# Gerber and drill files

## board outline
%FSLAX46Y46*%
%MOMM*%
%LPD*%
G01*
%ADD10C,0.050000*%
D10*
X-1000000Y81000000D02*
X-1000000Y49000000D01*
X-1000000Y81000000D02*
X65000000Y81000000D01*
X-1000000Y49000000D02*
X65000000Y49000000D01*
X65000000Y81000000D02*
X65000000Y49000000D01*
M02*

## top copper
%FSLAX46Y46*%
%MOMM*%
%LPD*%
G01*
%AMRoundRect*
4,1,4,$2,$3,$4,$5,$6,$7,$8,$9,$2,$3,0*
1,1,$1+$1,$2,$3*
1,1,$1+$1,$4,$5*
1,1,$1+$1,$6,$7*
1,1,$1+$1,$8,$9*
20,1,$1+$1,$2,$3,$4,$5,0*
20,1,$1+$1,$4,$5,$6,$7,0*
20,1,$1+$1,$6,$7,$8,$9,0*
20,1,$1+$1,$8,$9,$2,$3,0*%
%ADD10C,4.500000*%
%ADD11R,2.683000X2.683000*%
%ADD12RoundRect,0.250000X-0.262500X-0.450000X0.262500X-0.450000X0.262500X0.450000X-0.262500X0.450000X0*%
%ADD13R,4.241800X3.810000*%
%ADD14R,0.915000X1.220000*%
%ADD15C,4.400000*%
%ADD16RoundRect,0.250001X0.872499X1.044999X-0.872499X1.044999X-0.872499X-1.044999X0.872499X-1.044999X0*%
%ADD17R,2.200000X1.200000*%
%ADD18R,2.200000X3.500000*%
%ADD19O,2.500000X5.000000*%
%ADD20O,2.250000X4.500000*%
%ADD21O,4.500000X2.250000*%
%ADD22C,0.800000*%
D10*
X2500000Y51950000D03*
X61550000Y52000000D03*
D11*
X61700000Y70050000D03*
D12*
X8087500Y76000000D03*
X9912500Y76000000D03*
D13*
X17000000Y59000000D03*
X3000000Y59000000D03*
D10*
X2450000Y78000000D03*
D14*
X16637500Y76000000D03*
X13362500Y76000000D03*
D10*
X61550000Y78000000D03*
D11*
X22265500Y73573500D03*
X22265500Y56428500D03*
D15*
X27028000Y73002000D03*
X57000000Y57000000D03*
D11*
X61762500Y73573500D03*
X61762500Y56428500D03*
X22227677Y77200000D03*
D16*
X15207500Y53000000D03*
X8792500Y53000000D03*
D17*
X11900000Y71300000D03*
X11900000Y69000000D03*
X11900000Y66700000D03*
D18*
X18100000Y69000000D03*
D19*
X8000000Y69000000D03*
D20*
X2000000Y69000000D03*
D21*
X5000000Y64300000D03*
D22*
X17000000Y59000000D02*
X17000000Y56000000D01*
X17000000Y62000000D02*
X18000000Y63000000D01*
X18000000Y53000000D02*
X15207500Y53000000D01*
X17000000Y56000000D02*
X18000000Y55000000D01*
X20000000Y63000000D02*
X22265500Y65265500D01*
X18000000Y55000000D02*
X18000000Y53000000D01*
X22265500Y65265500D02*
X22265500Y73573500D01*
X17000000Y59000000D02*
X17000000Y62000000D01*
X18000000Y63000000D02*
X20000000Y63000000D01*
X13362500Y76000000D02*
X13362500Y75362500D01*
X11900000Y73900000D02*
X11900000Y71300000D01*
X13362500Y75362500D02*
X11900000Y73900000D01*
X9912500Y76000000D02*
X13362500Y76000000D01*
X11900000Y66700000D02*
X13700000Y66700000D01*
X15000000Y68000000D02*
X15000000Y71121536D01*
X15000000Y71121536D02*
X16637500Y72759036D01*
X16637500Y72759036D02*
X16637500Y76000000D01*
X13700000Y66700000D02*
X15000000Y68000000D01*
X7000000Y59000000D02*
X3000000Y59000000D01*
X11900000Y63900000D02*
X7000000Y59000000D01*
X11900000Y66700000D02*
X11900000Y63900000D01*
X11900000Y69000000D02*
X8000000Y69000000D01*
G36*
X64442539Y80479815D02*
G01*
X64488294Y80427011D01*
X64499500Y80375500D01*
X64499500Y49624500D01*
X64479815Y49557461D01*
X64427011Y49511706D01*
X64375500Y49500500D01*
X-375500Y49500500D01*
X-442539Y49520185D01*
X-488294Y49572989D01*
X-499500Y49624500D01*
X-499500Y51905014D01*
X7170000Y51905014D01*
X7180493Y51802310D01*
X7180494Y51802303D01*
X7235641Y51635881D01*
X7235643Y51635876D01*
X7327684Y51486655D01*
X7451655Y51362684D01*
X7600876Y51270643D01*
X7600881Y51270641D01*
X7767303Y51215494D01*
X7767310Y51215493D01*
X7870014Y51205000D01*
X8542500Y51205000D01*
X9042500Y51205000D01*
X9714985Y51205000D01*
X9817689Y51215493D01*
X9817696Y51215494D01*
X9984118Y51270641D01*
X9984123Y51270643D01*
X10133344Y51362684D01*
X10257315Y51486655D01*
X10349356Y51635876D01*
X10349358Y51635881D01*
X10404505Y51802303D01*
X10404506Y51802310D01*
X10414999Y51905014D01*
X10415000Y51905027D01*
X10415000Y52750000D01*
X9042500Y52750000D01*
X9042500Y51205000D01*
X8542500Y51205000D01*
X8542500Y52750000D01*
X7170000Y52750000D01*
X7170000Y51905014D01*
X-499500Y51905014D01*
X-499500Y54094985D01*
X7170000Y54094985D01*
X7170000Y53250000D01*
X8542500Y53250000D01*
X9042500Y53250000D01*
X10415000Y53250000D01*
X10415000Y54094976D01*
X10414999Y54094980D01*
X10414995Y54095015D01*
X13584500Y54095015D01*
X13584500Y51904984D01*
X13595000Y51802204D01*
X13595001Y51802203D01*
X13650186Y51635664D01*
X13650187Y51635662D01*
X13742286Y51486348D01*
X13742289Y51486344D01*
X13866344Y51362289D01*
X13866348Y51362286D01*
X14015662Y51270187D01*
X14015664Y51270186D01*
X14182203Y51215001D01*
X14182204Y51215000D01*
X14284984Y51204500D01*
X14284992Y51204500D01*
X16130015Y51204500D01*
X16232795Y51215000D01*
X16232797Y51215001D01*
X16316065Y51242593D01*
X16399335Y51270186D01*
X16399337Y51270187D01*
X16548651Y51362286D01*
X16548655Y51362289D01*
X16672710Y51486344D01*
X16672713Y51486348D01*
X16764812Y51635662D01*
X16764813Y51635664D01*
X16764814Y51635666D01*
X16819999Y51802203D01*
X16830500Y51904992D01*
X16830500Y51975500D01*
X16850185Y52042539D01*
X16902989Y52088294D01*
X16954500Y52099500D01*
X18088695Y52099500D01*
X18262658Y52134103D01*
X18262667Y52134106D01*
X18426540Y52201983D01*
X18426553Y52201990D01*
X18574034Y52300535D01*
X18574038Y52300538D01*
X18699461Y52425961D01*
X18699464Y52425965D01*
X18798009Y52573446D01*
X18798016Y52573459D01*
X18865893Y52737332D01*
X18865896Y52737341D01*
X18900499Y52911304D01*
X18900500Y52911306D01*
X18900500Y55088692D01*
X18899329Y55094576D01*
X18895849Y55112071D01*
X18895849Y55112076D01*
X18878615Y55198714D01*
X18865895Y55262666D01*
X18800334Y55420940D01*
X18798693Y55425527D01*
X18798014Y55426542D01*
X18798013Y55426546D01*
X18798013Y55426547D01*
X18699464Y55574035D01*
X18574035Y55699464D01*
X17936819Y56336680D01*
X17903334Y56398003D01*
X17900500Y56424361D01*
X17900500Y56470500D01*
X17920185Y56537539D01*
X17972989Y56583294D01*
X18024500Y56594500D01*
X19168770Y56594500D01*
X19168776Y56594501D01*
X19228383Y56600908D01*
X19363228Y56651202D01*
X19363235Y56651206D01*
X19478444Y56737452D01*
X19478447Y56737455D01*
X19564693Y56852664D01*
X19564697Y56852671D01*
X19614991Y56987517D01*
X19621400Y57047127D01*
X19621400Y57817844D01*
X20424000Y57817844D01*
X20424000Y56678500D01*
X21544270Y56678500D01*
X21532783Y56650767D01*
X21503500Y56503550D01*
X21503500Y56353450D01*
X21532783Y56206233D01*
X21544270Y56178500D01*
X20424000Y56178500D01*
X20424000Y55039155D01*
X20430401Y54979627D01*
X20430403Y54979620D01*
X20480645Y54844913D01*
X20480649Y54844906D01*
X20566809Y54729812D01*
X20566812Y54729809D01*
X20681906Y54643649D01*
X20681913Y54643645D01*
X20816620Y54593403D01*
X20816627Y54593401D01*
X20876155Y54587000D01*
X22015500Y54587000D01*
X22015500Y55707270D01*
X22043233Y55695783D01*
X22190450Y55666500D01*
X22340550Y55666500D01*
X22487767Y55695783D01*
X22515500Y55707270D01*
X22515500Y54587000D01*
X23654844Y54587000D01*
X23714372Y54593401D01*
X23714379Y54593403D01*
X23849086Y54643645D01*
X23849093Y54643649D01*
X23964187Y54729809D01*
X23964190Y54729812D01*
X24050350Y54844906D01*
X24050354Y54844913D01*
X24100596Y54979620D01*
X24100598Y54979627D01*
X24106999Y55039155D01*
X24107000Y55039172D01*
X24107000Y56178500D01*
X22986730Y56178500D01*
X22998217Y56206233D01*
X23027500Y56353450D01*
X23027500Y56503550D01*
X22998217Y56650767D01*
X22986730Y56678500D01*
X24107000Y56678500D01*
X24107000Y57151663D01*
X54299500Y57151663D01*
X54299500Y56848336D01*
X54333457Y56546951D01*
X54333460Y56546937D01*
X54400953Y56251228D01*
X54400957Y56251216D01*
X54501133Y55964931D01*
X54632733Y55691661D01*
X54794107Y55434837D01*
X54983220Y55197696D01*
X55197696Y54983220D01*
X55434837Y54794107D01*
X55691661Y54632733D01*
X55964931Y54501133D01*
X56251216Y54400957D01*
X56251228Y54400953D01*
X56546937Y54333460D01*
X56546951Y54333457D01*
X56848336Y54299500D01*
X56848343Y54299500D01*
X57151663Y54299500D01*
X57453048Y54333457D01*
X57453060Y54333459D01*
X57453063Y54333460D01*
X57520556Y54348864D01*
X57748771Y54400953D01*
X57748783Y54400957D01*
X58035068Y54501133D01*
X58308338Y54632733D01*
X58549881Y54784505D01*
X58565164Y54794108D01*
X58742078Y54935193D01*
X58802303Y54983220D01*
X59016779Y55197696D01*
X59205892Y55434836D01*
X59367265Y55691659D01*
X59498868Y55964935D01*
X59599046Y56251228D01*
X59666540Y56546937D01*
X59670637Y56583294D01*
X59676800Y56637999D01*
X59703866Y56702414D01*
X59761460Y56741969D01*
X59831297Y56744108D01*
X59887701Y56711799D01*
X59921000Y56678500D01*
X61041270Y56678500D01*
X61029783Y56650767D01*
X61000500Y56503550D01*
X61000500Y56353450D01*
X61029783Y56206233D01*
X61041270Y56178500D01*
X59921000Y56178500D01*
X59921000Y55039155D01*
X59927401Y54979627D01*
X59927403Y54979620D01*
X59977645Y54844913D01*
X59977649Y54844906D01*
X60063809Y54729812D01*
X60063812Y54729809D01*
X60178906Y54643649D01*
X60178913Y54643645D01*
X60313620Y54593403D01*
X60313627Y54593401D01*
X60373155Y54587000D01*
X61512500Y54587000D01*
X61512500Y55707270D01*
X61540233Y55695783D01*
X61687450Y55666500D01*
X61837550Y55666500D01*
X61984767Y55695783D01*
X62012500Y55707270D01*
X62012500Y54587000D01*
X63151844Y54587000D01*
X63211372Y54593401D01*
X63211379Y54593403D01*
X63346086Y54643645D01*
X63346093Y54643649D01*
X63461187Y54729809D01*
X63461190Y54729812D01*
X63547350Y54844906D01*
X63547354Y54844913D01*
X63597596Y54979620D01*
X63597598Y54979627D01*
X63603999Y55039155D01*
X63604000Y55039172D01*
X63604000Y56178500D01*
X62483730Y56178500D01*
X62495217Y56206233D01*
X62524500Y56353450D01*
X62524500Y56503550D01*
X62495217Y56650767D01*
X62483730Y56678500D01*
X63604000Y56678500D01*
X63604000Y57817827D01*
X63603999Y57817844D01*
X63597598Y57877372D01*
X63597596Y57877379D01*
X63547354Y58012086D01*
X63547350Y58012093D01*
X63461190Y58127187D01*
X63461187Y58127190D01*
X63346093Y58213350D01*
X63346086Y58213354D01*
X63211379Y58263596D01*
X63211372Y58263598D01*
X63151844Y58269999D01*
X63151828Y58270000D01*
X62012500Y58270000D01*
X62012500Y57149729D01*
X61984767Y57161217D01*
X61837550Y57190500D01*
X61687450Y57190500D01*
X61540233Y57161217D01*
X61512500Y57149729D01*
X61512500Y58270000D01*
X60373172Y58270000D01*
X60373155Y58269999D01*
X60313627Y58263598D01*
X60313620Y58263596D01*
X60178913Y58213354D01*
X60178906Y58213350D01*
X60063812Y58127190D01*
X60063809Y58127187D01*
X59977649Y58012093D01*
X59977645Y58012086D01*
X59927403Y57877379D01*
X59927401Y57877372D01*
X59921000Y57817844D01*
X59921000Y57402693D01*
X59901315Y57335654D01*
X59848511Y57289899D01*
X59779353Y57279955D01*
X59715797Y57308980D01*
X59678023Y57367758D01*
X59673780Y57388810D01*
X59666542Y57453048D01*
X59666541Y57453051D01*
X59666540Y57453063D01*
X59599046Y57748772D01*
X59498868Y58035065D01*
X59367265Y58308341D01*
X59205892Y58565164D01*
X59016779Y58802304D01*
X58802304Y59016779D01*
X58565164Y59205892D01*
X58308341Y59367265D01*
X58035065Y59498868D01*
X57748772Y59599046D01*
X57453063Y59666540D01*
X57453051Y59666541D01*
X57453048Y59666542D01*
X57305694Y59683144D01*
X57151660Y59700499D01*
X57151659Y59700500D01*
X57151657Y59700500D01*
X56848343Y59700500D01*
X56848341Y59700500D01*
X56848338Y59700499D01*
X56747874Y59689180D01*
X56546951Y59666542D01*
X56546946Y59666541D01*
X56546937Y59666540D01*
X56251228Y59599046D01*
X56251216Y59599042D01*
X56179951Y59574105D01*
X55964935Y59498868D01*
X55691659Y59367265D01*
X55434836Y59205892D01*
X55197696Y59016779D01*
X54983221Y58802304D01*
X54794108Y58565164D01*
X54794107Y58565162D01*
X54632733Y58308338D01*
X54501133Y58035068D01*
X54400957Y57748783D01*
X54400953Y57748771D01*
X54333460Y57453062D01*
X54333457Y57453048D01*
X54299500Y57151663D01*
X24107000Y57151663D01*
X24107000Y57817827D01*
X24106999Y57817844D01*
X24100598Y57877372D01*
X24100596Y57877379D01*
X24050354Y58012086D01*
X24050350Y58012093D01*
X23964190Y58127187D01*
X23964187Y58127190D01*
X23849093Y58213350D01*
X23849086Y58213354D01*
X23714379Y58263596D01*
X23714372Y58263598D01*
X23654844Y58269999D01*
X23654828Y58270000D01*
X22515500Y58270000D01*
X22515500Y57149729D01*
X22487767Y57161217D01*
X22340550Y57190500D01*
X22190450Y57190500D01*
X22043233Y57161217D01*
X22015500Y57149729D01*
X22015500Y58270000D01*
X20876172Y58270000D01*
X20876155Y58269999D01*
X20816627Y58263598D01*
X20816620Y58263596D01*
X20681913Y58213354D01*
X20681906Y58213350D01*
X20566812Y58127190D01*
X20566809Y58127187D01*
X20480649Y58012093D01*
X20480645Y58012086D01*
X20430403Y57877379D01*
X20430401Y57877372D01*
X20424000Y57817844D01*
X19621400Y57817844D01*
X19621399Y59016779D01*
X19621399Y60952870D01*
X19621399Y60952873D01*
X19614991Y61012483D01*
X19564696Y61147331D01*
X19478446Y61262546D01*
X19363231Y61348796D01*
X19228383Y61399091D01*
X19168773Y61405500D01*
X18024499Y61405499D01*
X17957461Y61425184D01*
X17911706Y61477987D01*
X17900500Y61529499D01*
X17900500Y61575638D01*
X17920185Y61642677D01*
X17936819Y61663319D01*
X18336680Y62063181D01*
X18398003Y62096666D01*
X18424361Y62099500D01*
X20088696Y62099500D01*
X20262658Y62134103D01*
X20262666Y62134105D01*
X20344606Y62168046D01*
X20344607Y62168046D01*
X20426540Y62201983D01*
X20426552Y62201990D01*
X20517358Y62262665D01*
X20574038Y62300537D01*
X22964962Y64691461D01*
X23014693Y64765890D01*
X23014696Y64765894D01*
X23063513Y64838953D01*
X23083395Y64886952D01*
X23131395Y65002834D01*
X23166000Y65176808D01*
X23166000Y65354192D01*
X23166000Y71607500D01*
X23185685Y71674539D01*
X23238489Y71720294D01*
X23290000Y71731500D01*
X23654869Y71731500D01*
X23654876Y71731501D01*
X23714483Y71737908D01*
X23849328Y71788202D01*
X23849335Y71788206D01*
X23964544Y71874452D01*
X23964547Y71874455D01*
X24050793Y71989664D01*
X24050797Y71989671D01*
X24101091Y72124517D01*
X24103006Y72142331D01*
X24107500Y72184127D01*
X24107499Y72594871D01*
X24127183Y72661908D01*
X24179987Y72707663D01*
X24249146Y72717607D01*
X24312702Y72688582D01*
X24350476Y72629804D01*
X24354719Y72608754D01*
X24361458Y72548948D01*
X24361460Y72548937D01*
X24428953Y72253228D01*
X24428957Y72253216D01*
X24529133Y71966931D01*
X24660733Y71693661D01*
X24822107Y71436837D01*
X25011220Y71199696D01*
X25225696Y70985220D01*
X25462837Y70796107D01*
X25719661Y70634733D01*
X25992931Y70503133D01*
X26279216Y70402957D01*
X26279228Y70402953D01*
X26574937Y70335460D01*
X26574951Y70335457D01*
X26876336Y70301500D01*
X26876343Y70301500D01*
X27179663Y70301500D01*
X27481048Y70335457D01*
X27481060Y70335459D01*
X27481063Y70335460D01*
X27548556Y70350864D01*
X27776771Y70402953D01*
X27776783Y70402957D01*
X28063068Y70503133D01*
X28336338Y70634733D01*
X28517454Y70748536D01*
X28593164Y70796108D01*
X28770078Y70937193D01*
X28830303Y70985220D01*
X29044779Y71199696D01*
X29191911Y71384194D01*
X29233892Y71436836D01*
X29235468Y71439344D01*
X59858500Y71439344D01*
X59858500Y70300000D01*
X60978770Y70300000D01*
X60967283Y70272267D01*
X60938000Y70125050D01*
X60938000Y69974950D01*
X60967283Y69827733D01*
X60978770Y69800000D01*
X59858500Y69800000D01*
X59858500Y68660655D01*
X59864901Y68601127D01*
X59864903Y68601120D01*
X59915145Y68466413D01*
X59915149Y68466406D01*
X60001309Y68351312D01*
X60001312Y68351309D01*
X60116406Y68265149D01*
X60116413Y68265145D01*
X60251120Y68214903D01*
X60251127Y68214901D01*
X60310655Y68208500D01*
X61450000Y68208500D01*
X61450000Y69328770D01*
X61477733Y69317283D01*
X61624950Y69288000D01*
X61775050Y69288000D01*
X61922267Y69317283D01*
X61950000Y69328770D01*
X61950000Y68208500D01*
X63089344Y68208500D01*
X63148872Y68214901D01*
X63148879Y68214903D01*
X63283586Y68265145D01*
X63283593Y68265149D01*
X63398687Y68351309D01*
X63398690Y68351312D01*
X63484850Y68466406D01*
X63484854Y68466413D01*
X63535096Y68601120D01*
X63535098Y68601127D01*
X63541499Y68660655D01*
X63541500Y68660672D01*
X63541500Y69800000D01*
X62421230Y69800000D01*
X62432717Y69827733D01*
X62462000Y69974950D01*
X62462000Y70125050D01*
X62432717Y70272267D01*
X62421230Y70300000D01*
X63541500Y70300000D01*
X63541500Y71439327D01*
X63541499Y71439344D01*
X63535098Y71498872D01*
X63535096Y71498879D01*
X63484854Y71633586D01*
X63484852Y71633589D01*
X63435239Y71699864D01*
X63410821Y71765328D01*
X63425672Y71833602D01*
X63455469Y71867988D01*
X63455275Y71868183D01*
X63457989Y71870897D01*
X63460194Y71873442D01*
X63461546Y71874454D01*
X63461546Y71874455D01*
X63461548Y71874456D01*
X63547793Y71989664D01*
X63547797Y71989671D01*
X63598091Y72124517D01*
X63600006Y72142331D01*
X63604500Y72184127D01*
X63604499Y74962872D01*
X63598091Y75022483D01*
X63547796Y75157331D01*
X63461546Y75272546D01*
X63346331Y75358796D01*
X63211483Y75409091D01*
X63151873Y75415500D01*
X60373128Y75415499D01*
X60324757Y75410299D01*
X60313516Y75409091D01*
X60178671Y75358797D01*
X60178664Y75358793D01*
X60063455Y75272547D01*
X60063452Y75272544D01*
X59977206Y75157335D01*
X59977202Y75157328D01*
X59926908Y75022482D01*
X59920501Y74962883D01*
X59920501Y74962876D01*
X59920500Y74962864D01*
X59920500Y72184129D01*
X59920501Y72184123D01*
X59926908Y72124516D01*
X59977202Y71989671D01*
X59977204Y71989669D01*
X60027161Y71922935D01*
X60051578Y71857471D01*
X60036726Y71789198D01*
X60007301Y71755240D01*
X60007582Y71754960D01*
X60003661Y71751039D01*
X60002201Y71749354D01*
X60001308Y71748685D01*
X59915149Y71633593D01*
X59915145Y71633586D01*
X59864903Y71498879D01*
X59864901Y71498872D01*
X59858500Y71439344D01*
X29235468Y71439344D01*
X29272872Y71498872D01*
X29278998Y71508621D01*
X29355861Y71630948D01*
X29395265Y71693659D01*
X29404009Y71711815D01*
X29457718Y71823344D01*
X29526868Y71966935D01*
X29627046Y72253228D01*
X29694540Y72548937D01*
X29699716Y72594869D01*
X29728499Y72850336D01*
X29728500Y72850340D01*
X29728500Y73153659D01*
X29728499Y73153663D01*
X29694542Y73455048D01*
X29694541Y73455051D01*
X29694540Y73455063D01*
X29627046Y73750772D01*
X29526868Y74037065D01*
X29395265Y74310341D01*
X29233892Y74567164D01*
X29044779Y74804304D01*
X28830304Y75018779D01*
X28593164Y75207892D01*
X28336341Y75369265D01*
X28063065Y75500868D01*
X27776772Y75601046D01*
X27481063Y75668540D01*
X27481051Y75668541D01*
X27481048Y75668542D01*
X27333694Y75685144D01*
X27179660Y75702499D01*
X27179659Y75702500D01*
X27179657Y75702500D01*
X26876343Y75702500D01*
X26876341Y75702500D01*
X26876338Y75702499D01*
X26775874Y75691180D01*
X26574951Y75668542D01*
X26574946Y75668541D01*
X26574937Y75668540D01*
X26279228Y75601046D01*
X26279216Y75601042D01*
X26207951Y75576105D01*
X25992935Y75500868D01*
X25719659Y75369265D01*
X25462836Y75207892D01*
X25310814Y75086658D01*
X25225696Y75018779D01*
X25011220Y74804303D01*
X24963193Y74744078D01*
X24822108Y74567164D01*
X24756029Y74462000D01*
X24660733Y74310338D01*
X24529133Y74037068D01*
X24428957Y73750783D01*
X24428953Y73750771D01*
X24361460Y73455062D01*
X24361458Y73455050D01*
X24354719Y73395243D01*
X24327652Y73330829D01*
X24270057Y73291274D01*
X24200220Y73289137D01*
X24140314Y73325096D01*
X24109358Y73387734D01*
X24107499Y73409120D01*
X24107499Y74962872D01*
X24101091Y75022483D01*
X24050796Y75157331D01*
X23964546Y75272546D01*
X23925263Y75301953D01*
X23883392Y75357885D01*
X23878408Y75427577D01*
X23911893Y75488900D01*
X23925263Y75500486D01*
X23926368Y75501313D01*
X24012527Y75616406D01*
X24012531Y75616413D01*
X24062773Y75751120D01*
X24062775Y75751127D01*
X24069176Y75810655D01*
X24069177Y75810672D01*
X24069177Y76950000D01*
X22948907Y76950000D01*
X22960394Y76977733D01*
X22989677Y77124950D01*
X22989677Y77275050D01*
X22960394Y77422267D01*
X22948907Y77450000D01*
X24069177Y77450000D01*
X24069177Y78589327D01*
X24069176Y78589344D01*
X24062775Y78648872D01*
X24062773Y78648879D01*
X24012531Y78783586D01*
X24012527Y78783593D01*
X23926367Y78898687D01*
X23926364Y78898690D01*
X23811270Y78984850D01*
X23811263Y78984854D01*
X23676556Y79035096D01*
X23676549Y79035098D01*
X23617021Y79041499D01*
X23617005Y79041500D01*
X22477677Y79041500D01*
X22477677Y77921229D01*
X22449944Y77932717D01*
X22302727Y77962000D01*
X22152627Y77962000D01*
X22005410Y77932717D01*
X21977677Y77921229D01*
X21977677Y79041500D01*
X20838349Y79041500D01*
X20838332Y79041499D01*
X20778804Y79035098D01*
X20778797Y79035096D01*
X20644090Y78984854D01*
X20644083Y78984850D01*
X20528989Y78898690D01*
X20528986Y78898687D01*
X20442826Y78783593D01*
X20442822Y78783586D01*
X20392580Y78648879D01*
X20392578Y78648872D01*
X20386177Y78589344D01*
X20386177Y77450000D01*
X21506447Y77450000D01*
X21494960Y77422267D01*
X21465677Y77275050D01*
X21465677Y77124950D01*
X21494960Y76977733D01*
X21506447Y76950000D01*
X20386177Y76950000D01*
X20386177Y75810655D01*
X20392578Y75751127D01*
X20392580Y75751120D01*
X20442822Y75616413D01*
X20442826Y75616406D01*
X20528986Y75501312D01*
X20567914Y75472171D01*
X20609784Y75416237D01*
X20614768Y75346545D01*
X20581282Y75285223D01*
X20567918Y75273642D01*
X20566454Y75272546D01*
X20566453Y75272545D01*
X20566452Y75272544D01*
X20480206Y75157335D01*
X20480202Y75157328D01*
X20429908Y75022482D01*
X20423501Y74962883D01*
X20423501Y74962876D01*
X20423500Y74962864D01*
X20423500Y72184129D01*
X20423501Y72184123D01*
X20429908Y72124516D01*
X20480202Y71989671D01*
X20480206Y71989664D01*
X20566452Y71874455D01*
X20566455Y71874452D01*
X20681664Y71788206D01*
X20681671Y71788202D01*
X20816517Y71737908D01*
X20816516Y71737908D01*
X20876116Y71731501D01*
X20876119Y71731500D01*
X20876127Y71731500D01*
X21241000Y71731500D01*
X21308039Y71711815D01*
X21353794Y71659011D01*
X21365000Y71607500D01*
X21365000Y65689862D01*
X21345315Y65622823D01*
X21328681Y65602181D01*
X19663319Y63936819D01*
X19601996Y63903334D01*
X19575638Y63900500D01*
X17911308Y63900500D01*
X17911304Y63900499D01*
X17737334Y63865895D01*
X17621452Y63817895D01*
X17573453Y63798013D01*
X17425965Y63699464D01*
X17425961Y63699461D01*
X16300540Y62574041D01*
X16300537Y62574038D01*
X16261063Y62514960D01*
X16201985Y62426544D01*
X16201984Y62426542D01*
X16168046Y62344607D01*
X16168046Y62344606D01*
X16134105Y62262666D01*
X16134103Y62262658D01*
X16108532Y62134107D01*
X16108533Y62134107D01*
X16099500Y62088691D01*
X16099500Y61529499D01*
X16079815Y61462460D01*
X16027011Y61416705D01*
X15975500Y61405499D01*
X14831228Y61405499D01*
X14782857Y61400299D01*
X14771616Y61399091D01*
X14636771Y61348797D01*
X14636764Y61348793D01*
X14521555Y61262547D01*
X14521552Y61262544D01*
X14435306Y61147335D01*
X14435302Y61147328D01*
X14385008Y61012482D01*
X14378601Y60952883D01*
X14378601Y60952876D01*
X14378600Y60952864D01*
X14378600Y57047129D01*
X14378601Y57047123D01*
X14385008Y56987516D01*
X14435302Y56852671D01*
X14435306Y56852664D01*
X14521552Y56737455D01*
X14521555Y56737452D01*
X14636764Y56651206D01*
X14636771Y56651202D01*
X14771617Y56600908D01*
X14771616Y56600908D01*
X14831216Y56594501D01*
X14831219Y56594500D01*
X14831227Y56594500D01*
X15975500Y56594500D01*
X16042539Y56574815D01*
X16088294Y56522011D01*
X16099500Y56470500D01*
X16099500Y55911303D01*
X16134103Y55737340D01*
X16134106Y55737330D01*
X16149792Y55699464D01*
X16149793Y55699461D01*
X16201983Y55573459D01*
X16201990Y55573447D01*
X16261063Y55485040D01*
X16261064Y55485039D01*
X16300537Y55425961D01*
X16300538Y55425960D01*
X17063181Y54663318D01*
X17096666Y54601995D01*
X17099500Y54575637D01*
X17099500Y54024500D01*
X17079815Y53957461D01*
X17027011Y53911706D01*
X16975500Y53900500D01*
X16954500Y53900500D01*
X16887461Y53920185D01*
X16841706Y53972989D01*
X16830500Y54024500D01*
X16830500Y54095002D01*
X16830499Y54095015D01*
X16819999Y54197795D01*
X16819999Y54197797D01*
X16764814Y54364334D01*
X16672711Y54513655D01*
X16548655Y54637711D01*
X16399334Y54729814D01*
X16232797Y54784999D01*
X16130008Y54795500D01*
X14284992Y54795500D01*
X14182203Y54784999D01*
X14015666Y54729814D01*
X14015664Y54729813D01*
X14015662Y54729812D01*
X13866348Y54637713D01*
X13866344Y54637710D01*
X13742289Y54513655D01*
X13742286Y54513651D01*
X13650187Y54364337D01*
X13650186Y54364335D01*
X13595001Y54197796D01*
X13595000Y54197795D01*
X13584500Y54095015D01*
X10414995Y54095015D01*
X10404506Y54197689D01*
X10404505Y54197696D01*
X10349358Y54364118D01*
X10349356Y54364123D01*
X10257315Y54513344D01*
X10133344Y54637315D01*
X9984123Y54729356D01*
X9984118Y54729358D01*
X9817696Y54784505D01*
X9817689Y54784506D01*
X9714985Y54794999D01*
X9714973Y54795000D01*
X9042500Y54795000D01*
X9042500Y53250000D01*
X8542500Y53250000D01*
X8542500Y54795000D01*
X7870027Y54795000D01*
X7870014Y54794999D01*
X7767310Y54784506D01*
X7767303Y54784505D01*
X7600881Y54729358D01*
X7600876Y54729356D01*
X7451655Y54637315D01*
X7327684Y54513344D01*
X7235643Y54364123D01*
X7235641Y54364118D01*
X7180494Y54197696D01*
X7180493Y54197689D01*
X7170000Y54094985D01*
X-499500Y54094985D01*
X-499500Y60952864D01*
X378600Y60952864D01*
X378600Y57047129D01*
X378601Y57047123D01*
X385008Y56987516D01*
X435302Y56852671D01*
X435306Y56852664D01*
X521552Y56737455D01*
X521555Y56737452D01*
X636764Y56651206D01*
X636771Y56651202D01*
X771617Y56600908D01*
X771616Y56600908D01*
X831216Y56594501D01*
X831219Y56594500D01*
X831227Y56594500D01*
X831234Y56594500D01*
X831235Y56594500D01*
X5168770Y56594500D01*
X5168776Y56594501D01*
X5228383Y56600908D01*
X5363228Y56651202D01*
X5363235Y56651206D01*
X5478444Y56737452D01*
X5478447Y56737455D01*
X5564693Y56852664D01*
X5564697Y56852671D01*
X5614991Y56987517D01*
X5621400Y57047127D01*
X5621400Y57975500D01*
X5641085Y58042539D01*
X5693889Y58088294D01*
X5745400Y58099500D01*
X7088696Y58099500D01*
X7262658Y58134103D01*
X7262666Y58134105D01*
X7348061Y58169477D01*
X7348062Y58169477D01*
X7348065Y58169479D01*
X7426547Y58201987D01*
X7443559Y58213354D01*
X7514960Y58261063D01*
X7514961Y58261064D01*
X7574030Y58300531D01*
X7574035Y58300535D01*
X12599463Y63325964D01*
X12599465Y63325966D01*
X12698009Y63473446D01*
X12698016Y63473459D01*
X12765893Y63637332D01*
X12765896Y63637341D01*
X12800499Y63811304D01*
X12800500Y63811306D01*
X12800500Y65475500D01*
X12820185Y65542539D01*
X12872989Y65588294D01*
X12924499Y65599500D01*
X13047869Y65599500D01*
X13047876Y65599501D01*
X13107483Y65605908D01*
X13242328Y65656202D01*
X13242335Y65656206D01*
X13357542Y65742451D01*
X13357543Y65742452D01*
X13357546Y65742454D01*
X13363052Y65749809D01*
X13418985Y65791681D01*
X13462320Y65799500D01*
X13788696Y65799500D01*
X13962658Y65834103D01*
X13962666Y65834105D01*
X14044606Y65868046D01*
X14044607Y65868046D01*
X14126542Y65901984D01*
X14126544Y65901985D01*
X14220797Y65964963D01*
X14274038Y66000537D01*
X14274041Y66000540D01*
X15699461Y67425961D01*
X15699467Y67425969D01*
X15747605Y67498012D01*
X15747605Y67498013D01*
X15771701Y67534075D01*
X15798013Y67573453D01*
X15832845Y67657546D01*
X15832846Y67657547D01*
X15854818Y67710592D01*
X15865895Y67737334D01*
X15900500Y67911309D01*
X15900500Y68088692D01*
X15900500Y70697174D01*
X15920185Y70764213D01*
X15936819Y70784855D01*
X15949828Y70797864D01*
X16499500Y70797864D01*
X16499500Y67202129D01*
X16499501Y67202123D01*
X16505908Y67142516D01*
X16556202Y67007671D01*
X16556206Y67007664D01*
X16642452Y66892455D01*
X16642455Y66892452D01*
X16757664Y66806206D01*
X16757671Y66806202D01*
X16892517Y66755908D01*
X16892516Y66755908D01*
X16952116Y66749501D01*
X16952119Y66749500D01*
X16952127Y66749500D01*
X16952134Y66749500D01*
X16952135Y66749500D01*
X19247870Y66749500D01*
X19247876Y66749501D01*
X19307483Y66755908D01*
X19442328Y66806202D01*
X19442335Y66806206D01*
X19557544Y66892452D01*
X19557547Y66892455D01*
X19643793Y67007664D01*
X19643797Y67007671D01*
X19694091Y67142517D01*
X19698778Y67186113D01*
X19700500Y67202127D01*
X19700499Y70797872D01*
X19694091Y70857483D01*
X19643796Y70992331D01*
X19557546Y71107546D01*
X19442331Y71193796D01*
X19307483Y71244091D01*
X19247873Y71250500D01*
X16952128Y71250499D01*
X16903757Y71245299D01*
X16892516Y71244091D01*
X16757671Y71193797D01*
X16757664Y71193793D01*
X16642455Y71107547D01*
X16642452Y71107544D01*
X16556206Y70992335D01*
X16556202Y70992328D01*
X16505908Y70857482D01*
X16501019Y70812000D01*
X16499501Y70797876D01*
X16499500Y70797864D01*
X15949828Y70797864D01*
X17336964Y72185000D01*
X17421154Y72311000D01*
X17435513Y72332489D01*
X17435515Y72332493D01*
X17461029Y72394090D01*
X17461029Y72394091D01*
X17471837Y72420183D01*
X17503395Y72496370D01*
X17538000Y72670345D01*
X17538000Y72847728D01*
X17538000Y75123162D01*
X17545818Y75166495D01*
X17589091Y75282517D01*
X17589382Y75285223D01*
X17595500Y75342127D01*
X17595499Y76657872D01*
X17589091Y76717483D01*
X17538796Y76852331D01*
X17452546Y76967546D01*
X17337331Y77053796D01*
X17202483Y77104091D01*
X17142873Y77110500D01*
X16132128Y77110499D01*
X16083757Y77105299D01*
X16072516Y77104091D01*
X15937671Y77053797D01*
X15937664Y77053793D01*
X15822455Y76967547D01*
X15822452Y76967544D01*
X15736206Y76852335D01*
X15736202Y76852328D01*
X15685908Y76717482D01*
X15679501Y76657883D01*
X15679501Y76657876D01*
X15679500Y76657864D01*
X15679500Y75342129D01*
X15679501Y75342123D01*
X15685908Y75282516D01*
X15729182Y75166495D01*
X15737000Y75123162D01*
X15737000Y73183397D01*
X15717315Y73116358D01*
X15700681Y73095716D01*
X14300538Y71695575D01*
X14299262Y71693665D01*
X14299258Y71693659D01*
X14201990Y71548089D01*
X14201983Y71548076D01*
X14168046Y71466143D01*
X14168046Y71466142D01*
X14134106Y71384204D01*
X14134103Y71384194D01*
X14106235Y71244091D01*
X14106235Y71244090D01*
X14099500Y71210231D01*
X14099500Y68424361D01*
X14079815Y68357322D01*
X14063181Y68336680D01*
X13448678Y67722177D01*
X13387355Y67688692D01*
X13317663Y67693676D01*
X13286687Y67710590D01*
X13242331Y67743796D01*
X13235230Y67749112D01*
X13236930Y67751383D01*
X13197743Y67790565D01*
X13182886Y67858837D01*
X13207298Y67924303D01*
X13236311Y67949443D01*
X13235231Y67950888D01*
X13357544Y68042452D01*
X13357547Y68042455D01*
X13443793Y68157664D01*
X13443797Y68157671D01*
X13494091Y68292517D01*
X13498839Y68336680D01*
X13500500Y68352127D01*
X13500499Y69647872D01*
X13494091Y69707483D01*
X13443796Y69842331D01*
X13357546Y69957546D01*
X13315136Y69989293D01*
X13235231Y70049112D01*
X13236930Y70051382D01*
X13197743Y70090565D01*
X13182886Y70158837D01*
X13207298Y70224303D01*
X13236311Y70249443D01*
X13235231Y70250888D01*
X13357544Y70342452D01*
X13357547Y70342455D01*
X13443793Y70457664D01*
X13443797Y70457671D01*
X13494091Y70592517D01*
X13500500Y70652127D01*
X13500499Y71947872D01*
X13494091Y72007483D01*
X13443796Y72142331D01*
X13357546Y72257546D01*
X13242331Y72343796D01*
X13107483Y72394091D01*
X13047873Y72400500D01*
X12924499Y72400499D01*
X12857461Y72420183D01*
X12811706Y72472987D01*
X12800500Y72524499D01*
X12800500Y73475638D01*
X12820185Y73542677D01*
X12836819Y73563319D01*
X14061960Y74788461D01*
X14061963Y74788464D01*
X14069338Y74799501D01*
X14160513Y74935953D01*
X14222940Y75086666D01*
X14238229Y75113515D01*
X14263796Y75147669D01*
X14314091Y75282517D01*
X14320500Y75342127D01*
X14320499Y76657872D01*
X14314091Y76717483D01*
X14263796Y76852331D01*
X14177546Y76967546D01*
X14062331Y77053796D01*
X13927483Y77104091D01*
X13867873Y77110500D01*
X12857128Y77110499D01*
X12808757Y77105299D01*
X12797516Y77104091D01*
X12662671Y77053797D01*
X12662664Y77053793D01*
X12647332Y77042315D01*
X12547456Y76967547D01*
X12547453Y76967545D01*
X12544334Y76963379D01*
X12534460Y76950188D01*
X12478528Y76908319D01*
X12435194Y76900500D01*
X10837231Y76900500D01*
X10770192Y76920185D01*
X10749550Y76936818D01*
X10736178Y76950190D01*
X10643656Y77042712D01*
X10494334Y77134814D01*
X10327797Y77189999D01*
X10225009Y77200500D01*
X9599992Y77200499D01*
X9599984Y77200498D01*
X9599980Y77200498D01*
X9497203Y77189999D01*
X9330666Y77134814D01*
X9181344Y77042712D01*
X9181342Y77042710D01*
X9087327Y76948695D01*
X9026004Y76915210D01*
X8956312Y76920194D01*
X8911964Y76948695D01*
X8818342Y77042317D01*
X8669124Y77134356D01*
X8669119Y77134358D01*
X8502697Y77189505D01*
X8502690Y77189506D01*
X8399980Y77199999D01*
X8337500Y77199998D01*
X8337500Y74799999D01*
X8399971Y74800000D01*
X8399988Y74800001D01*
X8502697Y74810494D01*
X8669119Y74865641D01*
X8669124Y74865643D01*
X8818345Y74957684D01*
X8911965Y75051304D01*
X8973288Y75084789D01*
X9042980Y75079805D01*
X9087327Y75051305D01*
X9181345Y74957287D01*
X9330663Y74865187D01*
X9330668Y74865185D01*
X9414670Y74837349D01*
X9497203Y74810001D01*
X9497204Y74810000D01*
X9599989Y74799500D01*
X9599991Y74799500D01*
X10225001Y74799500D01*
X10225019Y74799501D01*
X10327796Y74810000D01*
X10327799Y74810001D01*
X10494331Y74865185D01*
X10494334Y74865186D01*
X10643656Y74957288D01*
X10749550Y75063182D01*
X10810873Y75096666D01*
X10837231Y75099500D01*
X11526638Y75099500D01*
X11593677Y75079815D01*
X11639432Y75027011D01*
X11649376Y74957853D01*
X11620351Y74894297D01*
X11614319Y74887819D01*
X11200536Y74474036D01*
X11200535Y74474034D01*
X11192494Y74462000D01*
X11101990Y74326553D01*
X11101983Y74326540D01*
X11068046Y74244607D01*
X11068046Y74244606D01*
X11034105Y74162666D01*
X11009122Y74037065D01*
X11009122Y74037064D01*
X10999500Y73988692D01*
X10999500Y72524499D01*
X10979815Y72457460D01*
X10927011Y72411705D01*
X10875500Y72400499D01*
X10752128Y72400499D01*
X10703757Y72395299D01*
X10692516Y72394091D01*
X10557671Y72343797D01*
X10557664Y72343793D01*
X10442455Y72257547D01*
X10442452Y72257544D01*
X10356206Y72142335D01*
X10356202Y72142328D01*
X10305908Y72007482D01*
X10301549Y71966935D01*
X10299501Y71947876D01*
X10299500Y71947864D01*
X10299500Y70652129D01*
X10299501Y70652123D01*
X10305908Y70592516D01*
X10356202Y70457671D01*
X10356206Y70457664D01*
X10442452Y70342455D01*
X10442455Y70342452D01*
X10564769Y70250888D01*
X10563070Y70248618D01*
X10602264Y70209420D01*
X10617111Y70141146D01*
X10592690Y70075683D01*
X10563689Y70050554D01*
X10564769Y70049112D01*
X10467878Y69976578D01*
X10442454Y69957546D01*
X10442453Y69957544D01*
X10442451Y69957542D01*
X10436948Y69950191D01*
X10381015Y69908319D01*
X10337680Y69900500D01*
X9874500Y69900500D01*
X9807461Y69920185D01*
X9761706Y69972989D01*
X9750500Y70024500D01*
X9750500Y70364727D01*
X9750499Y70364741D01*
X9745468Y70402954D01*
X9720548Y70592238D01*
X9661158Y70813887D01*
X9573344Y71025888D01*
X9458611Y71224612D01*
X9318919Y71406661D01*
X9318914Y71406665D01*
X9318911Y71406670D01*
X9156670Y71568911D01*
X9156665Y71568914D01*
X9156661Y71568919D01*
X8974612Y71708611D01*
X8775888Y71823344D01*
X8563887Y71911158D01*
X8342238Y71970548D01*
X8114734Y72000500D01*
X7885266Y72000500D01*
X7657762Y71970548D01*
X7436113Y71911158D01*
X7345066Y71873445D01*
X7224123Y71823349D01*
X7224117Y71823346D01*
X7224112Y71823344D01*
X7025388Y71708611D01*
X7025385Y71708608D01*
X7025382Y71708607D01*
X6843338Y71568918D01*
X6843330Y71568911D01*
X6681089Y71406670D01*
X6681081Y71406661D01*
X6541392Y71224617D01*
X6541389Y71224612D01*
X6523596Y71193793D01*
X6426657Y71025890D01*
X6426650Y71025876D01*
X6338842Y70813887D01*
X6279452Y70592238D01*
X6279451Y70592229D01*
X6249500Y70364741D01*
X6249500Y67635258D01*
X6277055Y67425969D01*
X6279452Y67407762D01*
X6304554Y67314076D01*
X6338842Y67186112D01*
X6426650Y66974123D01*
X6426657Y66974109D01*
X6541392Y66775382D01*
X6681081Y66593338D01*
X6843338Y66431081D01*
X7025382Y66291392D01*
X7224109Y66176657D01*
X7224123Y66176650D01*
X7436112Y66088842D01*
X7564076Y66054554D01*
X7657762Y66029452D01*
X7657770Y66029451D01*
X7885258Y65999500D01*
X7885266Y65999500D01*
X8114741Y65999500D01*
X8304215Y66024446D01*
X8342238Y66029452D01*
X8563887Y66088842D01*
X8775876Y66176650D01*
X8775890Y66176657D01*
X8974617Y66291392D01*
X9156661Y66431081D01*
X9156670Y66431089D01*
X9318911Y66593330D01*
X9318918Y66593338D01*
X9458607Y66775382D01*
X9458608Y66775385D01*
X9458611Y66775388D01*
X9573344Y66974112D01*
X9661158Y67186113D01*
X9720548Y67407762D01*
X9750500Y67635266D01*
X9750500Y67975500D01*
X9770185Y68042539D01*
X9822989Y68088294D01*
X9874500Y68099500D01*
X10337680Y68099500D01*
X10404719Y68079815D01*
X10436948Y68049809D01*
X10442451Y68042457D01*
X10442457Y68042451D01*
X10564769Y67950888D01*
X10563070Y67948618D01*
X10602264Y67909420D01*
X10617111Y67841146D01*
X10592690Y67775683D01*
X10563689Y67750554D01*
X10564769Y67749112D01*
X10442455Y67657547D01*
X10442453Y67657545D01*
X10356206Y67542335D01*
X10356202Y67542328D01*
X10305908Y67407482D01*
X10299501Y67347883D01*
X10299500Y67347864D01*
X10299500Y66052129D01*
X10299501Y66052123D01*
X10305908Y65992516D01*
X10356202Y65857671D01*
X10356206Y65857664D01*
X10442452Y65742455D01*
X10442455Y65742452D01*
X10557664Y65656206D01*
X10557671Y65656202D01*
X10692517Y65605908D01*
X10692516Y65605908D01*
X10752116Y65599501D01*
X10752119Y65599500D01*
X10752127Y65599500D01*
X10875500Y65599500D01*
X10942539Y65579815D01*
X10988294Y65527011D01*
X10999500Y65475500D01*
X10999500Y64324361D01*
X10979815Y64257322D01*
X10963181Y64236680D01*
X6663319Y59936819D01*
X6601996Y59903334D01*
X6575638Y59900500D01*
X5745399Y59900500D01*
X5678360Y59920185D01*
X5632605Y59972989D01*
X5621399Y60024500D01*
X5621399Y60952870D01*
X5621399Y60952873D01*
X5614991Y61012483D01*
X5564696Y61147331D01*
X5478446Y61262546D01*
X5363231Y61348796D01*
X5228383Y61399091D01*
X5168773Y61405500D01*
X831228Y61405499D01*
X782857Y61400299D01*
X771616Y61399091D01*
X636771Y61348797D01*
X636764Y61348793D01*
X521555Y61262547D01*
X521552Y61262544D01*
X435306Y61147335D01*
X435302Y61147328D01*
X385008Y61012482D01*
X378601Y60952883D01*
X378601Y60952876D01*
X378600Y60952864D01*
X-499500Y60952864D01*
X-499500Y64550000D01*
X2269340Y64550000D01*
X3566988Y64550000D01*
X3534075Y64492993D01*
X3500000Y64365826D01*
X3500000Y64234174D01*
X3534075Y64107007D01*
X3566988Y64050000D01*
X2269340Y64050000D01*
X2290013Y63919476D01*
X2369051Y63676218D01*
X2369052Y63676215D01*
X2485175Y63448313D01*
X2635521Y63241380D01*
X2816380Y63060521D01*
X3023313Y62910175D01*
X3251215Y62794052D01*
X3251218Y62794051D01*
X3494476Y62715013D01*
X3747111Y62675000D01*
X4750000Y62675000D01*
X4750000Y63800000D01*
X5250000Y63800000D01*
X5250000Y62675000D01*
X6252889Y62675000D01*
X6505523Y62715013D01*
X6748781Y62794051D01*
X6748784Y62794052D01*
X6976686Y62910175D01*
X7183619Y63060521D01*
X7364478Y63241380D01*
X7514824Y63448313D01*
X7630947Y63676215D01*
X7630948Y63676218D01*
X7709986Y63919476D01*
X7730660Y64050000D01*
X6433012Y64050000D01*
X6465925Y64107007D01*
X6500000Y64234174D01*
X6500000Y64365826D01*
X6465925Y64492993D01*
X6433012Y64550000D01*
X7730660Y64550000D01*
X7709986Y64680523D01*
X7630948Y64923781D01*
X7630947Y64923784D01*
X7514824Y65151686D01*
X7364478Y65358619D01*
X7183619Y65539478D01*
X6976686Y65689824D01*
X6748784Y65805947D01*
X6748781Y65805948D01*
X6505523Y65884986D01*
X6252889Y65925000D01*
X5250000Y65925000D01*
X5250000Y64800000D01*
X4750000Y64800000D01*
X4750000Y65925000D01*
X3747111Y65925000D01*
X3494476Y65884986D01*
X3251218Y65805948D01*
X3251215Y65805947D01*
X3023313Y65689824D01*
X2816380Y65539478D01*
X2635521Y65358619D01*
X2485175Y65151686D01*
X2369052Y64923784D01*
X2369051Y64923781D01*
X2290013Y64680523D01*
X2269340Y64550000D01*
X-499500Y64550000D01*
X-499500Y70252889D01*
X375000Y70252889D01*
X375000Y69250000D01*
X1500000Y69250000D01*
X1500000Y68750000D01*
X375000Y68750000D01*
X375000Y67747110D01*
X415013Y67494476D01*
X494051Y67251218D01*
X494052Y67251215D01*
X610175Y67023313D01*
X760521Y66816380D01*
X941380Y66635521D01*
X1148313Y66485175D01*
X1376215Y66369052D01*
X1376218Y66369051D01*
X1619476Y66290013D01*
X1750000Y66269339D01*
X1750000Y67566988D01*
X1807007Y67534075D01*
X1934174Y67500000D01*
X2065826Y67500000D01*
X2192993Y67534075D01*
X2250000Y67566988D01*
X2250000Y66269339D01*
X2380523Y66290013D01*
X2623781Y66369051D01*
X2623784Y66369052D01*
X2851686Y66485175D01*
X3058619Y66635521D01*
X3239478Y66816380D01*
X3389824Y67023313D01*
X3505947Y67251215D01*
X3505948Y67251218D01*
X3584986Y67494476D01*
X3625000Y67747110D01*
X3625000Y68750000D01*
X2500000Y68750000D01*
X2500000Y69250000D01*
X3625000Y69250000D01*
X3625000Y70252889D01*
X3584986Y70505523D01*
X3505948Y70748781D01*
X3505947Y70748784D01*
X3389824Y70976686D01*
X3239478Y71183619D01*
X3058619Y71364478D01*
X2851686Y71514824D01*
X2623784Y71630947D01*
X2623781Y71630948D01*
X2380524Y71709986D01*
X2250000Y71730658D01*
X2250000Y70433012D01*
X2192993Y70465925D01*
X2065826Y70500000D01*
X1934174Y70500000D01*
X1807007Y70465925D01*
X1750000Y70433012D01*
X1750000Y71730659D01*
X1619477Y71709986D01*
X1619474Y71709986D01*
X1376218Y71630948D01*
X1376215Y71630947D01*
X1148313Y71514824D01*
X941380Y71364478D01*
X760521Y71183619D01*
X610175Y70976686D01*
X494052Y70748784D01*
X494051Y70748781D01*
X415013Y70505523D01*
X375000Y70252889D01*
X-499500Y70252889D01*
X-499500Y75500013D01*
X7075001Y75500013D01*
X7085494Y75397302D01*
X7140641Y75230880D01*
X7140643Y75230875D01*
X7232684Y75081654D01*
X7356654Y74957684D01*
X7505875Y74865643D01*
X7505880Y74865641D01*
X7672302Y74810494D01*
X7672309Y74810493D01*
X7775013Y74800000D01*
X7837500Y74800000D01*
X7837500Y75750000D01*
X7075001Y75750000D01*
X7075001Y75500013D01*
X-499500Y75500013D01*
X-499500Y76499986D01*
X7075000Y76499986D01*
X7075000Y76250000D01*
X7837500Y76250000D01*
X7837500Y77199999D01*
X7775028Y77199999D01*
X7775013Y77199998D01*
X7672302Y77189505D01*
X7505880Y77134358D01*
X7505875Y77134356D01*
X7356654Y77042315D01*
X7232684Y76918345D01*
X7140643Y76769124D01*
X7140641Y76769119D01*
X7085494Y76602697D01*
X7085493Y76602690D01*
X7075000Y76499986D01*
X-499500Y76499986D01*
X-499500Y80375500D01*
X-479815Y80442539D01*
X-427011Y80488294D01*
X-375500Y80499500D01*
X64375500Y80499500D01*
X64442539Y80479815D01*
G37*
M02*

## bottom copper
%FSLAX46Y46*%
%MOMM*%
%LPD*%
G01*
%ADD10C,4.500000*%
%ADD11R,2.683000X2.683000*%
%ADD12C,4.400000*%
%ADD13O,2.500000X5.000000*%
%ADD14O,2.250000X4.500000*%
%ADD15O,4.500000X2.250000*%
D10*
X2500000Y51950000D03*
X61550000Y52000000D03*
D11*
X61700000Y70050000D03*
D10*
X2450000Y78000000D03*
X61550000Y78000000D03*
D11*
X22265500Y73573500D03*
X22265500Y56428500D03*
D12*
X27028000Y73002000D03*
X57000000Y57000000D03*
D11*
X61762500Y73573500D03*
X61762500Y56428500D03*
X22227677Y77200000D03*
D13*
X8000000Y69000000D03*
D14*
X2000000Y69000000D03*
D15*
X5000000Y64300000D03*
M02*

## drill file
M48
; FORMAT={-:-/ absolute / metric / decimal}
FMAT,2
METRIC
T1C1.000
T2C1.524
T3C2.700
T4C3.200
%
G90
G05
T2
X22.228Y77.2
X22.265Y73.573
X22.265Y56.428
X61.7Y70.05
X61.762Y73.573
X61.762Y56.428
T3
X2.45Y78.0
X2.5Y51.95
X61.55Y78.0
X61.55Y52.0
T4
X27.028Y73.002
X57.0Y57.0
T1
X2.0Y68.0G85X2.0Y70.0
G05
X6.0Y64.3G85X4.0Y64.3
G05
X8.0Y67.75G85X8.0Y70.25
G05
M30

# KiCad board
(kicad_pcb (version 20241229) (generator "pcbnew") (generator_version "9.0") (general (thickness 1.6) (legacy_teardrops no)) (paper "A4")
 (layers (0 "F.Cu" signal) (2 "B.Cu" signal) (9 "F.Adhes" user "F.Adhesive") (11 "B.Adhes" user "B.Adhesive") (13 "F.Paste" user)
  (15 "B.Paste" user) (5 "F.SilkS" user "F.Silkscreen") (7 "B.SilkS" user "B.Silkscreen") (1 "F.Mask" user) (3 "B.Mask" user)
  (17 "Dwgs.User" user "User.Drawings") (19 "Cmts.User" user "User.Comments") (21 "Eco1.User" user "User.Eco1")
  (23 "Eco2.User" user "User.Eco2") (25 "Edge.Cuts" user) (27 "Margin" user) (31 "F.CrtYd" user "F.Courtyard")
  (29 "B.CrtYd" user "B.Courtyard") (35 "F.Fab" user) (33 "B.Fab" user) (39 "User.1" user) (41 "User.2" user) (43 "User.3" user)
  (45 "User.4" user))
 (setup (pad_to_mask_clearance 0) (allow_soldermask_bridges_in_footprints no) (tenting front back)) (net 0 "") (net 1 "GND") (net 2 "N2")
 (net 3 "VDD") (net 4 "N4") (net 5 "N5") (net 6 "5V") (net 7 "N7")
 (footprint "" (layer "F.Cu") (at 2.5 -51.95)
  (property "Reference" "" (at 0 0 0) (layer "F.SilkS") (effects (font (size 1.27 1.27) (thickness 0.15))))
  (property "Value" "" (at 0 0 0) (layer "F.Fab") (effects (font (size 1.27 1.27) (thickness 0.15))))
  (pad "3" thru_hole circle (at 0 0) (size 4.5 4.5) (drill 2.7) (layers "*.Cu" "*.Mask") (remove_unused_layers no) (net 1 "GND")
   (zone_connect 2)))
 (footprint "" (layer "F.Cu") (at 61.55 -52)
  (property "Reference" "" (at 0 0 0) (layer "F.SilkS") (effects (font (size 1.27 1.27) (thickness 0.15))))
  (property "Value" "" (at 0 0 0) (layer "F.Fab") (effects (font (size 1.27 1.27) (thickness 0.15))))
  (pad "4" thru_hole circle (at 0 0) (size 4.5 4.5) (drill 2.7) (layers "*.Cu" "*.Mask") (remove_unused_layers no) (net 1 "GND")
   (zone_connect 2)))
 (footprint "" (layer "F.Cu") (at 61.7 -70.05)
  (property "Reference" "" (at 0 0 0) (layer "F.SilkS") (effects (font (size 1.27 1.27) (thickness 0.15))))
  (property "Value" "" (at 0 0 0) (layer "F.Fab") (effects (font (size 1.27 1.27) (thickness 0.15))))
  (pad "OUT-" thru_hole rect (at 0 0) (size 2.683 2.683) (drill 1.524) (layers "*.Cu" "*.Mask") (remove_unused_layers no) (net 1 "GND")
   (solder_mask_margin 0.102)))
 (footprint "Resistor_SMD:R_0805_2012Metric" (layer "F.Cu") (at 9 -76)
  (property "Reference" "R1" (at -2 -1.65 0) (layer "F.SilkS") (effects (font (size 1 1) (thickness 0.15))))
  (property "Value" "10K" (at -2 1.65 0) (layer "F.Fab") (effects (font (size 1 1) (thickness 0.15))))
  (pad "1" smd roundrect (at -0.9125 0) (size 1.025 1.4) (layers "F.Cu" "F.Mask" "F.Paste") (roundrect_rratio 0.243902) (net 1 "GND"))
  (pad "2" smd roundrect (at 0.9125 0) (size 1.025 1.4) (layers "F.Cu" "F.Mask" "F.Paste") (roundrect_rratio 0.243902) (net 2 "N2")))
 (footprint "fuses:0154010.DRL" (layer "F.Cu") (at 10 -59 180)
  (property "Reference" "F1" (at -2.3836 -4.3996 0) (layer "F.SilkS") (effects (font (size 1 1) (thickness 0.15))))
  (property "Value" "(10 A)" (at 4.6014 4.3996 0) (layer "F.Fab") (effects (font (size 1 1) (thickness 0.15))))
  (pad "1" smd rect (at -7 0 180) (size 4.2418 3.81) (layers "F.Cu" "F.Mask" "F.Paste") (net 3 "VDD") (solder_mask_margin 0.102))
  (pad "2" smd rect (at 7 0 180) (size 4.2418 3.81) (layers "F.Cu" "F.Mask" "F.Paste") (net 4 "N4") (solder_mask_margin 0.102)))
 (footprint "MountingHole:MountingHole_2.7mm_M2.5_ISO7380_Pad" (layer "F.Cu") (at 2.45 -78)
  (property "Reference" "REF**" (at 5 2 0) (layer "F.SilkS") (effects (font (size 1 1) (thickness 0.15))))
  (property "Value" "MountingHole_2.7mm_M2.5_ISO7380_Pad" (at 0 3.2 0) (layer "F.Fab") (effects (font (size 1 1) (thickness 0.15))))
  (pad "1" thru_hole circle (at 0 0) (size 4.5 4.5) (drill 2.7) (layers "*.Cu" "*.Mask") (remove_unused_layers no) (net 1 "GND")
   (zone_connect 2)))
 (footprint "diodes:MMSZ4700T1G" (layer "F.Cu") (at 15 -76 180)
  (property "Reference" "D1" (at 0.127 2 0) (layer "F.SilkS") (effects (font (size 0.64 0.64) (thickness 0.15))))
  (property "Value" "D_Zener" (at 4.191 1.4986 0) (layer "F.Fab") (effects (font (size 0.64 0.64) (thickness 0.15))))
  (pad "1" smd rect (at -1.6375 0 180) (size 0.915 1.22) (layers "F.Cu" "F.Mask" "F.Paste") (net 4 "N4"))
  (pad "2" smd rect (at 1.6375 0 180) (size 0.915 1.22) (layers "F.Cu" "F.Mask" "F.Paste") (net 2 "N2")))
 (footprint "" (layer "F.Cu") (at 61.55 -78)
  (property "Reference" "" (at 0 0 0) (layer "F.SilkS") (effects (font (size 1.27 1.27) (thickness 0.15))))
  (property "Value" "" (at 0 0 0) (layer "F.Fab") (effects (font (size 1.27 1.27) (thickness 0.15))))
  (pad "2" thru_hole circle (at 0 0) (size 4.5 4.5) (drill 2.7) (layers "*.Cu" "*.Mask") (remove_unused_layers no) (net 1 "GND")
   (zone_connect 2)))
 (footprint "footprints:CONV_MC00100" (layer "F.Cu") (at 42.014 -65.001)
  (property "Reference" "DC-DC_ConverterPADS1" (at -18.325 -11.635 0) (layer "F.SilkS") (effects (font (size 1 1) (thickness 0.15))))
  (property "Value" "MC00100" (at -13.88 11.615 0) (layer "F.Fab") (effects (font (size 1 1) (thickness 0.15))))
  (pad "IN+" thru_hole rect (at -19.7485 -8.5725) (size 2.683 2.683) (drill 1.524) (layers "*.Cu" "*.Mask") (remove_unused_layers no)
   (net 3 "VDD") (solder_mask_margin 0.102))
  (pad "IN-" thru_hole rect (at -19.7485 8.5725) (size 2.683 2.683) (drill 1.524) (layers "*.Cu" "*.Mask") (remove_unused_layers no)
   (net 1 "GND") (solder_mask_margin 0.102))
  (pad "MH1" thru_hole circle (at -14.986 -8.001) (size 4.4 4.4) (drill 3.2) (layers "*.Cu" "*.Mask") (remove_unused_layers no) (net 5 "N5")
   (solder_mask_margin 0.102))
  (pad "MH2" thru_hole circle (at 14.986 8.001) (size 4.4 4.4) (drill 3.2) (layers "*.Cu" "*.Mask") (remove_unused_layers no) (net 5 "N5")
   (solder_mask_margin 0.102))
  (pad "OUT+" thru_hole rect (at 19.7485 -8.5725) (size 2.683 2.683) (drill 1.524) (layers "*.Cu" "*.Mask") (remove_unused_layers no)
   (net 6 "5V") (solder_mask_margin 0.102))
  (pad "OUT-" thru_hole rect (at 19.7485 8.5725) (size 2.683 2.683) (drill 1.524) (layers "*.Cu" "*.Mask") (remove_unused_layers no)
   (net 1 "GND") (solder_mask_margin 0.102)))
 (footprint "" (layer "F.Cu") (at 22.227677 -77.2)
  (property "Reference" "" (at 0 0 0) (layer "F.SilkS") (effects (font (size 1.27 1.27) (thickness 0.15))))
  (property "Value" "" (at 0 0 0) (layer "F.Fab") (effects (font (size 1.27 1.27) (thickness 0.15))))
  (pad "OUT-" thru_hole rect (at 0 0) (size 2.683 2.683) (drill 1.524) (layers "*.Cu" "*.Mask") (remove_unused_layers no) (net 1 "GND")
   (solder_mask_margin 0.102)))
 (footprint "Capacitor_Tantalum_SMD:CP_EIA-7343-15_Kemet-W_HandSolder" (layer "F.Cu") (at 12 -53 180)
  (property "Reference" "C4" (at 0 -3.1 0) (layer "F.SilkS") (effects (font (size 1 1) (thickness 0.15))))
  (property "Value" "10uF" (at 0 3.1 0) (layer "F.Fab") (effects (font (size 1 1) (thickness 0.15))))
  (pad "1" smd roundrect (at -3.2075 0 180) (size 2.245 2.59) (layers "F.Cu" "F.Mask" "F.Paste") (roundrect_rratio 0.111359) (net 3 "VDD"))
  (pad "2" smd roundrect (at 3.2075 0 180) (size 2.245 2.59) (layers "F.Cu" "F.Mask" "F.Paste") (roundrect_rratio 0.111359) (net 1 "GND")))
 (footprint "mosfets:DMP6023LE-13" (layer "F.Cu") (at 15 -69)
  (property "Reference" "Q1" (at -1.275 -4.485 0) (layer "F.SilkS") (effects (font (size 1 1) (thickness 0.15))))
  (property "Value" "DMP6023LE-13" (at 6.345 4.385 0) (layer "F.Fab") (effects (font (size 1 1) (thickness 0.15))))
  (pad "1" smd rect (at -3.1 -2.3) (size 2.2 1.2) (layers "F.Cu" "F.Mask" "F.Paste") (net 2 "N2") (solder_mask_margin 0.102))
  (pad "2" smd rect (at -3.1 0) (size 2.2 1.2) (layers "F.Cu" "F.Mask" "F.Paste") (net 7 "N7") (solder_mask_margin 0.102))
  (pad "3" smd rect (at -3.1 2.3) (size 2.2 1.2) (layers "F.Cu" "F.Mask" "F.Paste") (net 4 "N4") (solder_mask_margin 0.102))
  (pad "4" smd rect (at 3.1 0) (size 2.2 3.5) (layers "F.Cu" "F.Mask" "F.Paste") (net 7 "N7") (solder_mask_margin 0.102)))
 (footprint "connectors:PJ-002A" (layer "F.Cu") (at 8 -69 180)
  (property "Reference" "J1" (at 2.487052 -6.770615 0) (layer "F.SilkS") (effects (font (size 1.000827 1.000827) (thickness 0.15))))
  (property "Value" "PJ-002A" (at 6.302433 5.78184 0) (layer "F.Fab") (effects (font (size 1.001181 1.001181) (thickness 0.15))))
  (pad "1" thru_hole oval (at 0 0 180) (size 2.5 5) (drill oval 1 3.5) (layers "*.Cu" "*.Mask") (remove_unused_layers no) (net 7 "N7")
   (solder_mask_margin 0.102))
  (pad "2" thru_hole oval (at 6 0 180) (size 2.25 4.5) (drill oval 1 3) (layers "*.Cu" "*.Mask") (remove_unused_layers no) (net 1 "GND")
   (solder_mask_margin 0.102))
  (pad "3" thru_hole oval (at 3 -4.7 180) (size 4.5 2.25) (drill oval 3 1) (layers "*.Cu" "*.Mask") (remove_unused_layers no) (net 1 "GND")
   (solder_mask_margin 0.102)))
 (gr_line (start -1 -81) (end -1 -49) (stroke (width 0.05) (type default)) (locked yes) (layer "Edge.Cuts"))
 (gr_line (start -1 -81) (end 65 -81) (stroke (width 0.05) (type solid)) (locked yes) (layer "Edge.Cuts"))
 (gr_line (start -1 -49) (end 65 -49) (stroke (width 0.05) (type solid)) (locked yes) (layer "Edge.Cuts"))
 (gr_line (start 65 -81) (end 65 -49) (stroke (width 0.05) (type default)) (locked yes) (layer "Edge.Cuts"))
 (segment (start 17 -59) (end 17 -56) (width 0.8) (layer "F.Cu") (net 3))
 (segment (start 17 -62) (end 18 -63) (width 0.8) (layer "F.Cu") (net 3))
 (segment (start 18 -53) (end 15.2075 -53) (width 0.8) (layer "F.Cu") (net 3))
 (segment (start 17 -56) (end 18 -55) (width 0.8) (layer "F.Cu") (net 3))
 (segment (start 20 -63) (end 22.2655 -65.2655) (width 0.8) (layer "F.Cu") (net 3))
 (segment (start 18 -55) (end 18 -53) (width 0.8) (layer "F.Cu") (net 3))
 (segment (start 22.2655 -65.2655) (end 22.2655 -73.5735) (width 0.8) (layer "F.Cu") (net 3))
 (segment (start 17 -59) (end 17 -62) (width 0.8) (layer "F.Cu") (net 3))
 (segment (start 18 -63) (end 20 -63) (width 0.8) (layer "F.Cu") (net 3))
 (segment (start 13.3625 -76) (end 13.3625 -75.3625) (width 0.8) (layer "F.Cu") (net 2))
 (segment (start 11.9 -73.9) (end 11.9 -71.3) (width 0.8) (layer "F.Cu") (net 2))
 (segment (start 13.3625 -75.3625) (end 11.9 -73.9) (width 0.8) (layer "F.Cu") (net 2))
 (segment (start 9.9125 -76) (end 13.3625 -76) (width 0.8) (layer "F.Cu") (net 2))
 (segment (start 11.9 -66.7) (end 13.7 -66.7) (width 0.8) (layer "F.Cu") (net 4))
 (segment (start 15 -68) (end 15 -71.121536) (width 0.8) (layer "F.Cu") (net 4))
 (segment (start 15 -71.121536) (end 16.6375 -72.759036) (width 0.8) (layer "F.Cu") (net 4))
 (segment (start 16.6375 -72.759036) (end 16.6375 -76) (width 0.8) (layer "F.Cu") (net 4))
 (segment (start 13.7 -66.7) (end 15 -68) (width 0.8) (layer "F.Cu") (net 4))
 (segment (start 7 -59) (end 3 -59) (width 0.8) (layer "F.Cu") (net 4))
 (segment (start 11.9 -63.9) (end 7 -59) (width 0.8) (layer "F.Cu") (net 4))
 (segment (start 11.9 -66.7) (end 11.9 -63.9) (width 0.8) (layer "F.Cu") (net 4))
 (segment (start 11.9 -69) (end 8 -69) (width 0.8) (layer "F.Cu") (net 7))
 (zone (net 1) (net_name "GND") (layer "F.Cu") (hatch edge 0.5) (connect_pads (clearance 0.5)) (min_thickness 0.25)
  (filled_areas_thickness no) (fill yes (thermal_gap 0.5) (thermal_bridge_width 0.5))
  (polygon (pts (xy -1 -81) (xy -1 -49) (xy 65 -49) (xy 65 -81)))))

